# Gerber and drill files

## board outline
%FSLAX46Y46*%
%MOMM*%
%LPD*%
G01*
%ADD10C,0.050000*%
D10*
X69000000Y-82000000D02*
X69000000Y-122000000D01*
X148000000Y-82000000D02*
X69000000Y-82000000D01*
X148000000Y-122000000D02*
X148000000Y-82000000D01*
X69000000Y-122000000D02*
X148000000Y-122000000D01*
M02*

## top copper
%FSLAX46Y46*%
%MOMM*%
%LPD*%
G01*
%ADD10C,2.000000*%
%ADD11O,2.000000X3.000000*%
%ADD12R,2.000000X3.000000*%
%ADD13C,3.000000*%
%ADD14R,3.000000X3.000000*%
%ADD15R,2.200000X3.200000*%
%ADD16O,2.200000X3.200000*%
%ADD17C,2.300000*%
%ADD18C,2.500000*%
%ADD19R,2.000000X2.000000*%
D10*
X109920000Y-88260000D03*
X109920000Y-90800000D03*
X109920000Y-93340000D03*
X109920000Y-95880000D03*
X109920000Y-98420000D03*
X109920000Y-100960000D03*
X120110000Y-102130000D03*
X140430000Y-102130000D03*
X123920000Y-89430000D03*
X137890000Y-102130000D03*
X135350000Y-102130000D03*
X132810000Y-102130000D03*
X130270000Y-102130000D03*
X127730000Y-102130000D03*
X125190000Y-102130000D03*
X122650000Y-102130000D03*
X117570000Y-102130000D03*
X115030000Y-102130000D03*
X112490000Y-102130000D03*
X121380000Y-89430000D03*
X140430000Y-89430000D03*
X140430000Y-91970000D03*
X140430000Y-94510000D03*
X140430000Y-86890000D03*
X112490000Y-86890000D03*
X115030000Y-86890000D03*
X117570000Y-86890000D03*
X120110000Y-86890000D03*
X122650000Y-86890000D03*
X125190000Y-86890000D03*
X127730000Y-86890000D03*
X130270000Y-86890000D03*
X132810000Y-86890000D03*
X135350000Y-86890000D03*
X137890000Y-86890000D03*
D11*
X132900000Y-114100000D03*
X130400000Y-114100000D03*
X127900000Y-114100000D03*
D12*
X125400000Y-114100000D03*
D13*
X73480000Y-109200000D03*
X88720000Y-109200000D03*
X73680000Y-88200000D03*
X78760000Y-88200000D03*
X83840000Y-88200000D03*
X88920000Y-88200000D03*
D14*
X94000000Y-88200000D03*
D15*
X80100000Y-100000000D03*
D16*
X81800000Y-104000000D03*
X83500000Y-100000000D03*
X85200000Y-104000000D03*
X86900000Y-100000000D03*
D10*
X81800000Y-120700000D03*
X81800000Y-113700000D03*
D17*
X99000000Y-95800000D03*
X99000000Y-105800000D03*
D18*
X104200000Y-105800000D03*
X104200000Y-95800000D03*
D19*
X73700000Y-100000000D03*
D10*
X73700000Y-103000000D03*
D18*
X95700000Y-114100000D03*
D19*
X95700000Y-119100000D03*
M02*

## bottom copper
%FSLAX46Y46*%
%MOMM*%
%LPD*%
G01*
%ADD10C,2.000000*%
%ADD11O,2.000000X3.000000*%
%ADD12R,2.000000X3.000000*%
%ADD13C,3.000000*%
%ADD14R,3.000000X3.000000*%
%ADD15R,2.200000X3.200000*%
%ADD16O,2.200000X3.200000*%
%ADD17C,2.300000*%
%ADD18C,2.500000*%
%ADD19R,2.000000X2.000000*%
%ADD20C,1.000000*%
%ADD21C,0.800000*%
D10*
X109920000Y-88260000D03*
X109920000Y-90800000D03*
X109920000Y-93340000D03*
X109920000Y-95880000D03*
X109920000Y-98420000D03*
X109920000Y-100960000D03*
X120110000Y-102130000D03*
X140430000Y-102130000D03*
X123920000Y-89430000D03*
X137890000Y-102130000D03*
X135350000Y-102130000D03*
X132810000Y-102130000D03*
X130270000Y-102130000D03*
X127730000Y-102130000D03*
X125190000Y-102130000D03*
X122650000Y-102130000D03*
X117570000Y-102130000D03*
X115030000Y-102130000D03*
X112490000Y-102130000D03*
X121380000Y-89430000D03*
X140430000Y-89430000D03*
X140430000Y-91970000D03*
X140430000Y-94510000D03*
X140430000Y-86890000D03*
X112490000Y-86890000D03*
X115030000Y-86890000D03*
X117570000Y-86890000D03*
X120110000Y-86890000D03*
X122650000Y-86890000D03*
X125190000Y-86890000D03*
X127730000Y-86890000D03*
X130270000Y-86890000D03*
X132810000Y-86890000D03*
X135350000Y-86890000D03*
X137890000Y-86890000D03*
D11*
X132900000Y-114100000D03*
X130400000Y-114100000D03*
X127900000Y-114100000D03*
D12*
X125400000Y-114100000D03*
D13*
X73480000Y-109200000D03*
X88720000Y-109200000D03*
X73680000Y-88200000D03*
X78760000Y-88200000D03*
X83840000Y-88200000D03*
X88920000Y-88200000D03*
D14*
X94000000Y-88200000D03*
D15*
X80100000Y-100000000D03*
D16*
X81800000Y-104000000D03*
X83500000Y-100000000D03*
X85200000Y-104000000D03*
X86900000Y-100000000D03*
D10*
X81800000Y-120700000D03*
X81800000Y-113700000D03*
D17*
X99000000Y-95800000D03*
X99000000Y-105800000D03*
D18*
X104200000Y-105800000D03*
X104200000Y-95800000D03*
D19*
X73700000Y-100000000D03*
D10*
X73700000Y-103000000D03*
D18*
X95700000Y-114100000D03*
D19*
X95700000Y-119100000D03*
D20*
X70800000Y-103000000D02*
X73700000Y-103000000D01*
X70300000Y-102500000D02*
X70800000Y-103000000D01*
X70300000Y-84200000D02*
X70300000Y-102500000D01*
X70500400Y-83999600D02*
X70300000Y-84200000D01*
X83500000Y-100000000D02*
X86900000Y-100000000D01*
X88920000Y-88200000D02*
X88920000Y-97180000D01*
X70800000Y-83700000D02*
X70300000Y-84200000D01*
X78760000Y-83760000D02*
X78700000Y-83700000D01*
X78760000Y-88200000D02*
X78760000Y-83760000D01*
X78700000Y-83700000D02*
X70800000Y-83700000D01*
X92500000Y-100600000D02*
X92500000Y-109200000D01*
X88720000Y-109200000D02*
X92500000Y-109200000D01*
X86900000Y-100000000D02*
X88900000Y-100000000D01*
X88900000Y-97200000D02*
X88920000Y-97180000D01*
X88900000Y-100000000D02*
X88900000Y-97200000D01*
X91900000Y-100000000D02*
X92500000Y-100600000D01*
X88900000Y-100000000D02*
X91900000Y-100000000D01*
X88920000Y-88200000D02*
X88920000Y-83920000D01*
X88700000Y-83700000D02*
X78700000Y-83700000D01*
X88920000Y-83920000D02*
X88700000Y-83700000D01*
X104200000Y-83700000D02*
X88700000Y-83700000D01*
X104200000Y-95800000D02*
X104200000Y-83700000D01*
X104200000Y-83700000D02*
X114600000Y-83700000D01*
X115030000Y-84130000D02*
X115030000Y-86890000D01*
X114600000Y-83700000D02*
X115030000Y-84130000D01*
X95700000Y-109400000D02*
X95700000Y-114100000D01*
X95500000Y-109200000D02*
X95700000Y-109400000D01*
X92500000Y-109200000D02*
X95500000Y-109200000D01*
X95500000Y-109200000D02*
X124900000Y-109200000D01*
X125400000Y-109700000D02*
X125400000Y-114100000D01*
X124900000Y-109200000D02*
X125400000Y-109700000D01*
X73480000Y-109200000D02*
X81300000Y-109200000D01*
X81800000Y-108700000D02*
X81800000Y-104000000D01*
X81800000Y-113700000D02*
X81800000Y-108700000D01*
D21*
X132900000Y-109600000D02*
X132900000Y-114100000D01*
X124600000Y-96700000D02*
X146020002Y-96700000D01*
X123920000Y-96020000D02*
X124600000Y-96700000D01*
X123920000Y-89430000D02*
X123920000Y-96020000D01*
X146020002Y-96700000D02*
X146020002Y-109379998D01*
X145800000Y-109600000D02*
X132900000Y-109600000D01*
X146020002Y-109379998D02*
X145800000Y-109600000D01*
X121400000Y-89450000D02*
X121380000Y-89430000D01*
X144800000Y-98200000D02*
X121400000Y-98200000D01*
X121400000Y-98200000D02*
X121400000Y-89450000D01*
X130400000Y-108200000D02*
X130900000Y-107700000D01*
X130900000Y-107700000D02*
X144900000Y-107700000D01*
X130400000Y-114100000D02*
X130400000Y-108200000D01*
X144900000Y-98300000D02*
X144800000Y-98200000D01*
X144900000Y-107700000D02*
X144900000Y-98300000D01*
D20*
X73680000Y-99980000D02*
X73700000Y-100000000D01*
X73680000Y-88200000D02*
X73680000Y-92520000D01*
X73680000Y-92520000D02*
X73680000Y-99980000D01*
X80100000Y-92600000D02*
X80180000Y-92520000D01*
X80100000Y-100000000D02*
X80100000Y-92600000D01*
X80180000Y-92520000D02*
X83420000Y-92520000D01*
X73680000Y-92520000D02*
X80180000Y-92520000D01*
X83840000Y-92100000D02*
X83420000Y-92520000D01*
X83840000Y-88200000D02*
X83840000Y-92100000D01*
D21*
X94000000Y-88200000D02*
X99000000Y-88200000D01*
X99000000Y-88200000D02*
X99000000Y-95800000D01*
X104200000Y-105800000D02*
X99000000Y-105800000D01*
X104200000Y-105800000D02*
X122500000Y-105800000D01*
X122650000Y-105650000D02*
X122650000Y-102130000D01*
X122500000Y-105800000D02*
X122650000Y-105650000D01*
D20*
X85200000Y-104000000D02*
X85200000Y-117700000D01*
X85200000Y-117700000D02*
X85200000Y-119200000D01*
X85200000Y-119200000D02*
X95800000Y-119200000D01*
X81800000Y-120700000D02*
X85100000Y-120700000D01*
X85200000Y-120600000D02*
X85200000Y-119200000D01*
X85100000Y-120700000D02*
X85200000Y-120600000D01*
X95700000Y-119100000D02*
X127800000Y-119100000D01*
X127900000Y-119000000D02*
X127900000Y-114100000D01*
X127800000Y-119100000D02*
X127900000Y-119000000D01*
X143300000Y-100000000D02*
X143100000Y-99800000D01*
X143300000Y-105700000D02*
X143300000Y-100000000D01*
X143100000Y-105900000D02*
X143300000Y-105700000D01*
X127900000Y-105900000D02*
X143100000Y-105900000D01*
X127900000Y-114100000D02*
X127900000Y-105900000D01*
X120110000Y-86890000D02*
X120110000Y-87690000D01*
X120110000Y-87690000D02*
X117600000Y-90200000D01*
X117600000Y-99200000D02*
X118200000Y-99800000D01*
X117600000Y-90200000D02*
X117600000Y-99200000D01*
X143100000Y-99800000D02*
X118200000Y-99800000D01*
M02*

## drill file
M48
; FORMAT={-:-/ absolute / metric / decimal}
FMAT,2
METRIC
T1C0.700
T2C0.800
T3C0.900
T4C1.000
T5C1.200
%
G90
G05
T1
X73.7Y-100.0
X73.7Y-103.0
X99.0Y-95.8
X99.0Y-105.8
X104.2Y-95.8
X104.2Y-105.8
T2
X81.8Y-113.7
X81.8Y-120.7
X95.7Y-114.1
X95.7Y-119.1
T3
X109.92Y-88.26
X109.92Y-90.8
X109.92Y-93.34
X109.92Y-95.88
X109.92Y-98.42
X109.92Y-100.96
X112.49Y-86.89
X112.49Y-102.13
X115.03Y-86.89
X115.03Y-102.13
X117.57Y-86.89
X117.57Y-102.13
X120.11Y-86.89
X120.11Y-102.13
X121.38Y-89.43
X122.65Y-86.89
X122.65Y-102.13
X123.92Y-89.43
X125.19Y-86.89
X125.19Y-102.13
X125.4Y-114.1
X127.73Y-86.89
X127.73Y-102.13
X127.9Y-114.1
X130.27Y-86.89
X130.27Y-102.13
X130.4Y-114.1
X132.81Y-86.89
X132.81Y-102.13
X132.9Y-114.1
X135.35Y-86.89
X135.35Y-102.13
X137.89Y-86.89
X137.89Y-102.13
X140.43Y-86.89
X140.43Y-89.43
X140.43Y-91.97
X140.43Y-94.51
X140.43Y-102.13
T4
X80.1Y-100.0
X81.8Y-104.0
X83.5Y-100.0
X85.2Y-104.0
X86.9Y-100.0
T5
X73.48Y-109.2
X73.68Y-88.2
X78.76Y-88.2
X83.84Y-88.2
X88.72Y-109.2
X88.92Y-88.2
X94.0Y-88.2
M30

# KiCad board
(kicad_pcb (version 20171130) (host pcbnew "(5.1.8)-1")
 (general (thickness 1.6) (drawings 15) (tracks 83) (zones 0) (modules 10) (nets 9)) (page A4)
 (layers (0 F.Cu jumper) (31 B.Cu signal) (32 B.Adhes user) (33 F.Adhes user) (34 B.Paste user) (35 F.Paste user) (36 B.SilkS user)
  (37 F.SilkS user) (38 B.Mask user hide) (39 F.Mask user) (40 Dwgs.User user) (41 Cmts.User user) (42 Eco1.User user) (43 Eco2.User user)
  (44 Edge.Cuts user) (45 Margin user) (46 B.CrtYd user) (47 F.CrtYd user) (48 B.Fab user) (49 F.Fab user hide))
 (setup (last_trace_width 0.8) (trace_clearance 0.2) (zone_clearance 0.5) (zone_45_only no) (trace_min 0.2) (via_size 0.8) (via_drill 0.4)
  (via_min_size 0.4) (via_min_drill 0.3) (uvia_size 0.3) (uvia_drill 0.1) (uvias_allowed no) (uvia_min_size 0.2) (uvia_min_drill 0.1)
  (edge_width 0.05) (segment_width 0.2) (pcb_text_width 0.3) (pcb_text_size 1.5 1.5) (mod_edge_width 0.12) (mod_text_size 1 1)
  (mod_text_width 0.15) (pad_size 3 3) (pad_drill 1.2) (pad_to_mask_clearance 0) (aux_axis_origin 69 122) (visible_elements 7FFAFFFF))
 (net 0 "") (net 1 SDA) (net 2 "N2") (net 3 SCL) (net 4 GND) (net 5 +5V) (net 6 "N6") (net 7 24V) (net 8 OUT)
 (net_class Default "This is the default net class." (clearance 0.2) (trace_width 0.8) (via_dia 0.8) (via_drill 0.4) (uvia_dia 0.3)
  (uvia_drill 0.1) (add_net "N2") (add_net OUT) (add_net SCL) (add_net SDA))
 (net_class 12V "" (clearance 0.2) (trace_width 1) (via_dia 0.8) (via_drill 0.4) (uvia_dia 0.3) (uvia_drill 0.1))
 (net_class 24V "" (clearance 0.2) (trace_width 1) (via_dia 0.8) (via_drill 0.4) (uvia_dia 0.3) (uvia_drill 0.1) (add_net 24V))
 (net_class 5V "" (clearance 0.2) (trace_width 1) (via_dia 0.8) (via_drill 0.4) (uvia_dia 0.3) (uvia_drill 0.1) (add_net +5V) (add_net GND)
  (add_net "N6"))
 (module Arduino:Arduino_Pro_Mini (layer F.Cu) (at 141.7 103.4 90)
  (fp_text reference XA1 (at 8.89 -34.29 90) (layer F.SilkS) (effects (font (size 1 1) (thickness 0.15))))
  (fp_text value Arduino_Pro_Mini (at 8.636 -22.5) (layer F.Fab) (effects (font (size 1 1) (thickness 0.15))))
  (pad GND5 thru_hole circle (at 15.14 -31.78 90) (size 2 2) (drill 0.9) (layers *.Cu *.Mask))
  (pad GND4 thru_hole circle (at 12.6 -31.78 90) (size 2 2) (drill 0.9) (layers *.Cu *.Mask))
  (pad VCC1 thru_hole circle (at 10.06 -31.78 90) (size 2 2) (drill 0.9) (layers *.Cu *.Mask))
  (pad RXI thru_hole circle (at 7.52 -31.78 90) (size 2 2) (drill 0.9) (layers *.Cu *.Mask))
  (pad TX0 thru_hole circle (at 4.98 -31.78 90) (size 2 2) (drill 0.9) (layers *.Cu *.Mask))
  (pad DTR thru_hole circle (at 2.44 -31.78 90) (size 2 2) (drill 0.9) (layers *.Cu *.Mask))
  (pad GND2 thru_hole circle (at 1.27 -21.59 90) (size 2 2) (drill 0.9) (layers *.Cu *.Mask))
  (pad D9 thru_hole circle (at 1.27 -1.27 90) (size 2 2) (drill 0.9) (layers *.Cu *.Mask))
  (pad A4 thru_hole circle (at 13.97 -17.78 90) (size 2 2) (drill 0.9) (layers *.Cu *.Mask) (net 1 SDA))
  (pad D8 thru_hole circle (at 1.27 -3.81 90) (size 2 2) (drill 0.9) (layers *.Cu *.Mask))
  (pad D7 thru_hole circle (at 1.27 -6.35 90) (size 2 2) (drill 0.9) (layers *.Cu *.Mask))
  (pad D6 thru_hole circle (at 1.27 -8.89 90) (size 2 2) (drill 0.9) (layers *.Cu *.Mask))
  (pad D5 thru_hole circle (at 1.27 -11.43 90) (size 2 2) (drill 0.9) (layers *.Cu *.Mask))
  (pad D4 thru_hole circle (at 1.27 -13.97 90) (size 2 2) (drill 0.9) (layers *.Cu *.Mask))
  (pad D3 thru_hole circle (at 1.27 -16.51 90) (size 2 2) (drill 0.9) (layers *.Cu *.Mask))
  (pad D2 thru_hole circle (at 1.27 -19.05 90) (size 2 2) (drill 0.9) (layers *.Cu *.Mask) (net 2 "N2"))
  (pad RST2 thru_hole circle (at 1.27 -24.13 90) (size 2 2) (drill 0.9) (layers *.Cu *.Mask))
  (pad D1 thru_hole circle (at 1.27 -26.67 90) (size 2 2) (drill 0.9) (layers *.Cu *.Mask))
  (pad D0 thru_hole circle (at 1.27 -29.21 90) (size 2 2) (drill 0.9) (layers *.Cu *.Mask))
  (pad A5 thru_hole circle (at 13.97 -20.32 90) (size 2 2) (drill 0.9) (layers *.Cu *.Mask) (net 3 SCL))
  (pad A7 thru_hole circle (at 13.97 -1.27 90) (size 2 2) (drill 0.9) (layers *.Cu *.Mask))
  (pad A6 thru_hole circle (at 11.43 -1.27 90) (size 2 2) (drill 0.9) (layers *.Cu *.Mask))
  (pad GND3 thru_hole circle (at 8.89 -1.27 90) (size 2 2) (drill 0.9) (layers *.Cu *.Mask))
  (pad D10 thru_hole circle (at 16.51 -1.27 90) (size 2 2) (drill 0.9) (layers *.Cu *.Mask))
  (pad RAW thru_hole circle (at 16.51 -29.21 90) (size 2 2) (drill 0.9) (layers *.Cu *.Mask))
  (pad GND thru_hole circle (at 16.51 -26.67 90) (size 2 2) (drill 0.9) (layers *.Cu *.Mask) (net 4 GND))
  (pad RST thru_hole circle (at 16.51 -24.13 90) (size 2 2) (drill 0.9) (layers *.Cu *.Mask))
  (pad VCC thru_hole circle (at 16.51 -21.59 90) (size 2 2) (drill 0.9) (layers *.Cu *.Mask) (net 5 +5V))
  (pad A3 thru_hole circle (at 16.51 -19.05 90) (size 2 2) (drill 0.9) (layers *.Cu *.Mask))
  (pad A2 thru_hole circle (at 16.51 -16.51 90) (size 2 2) (drill 0.9) (layers *.Cu *.Mask))
  (pad A1 thru_hole circle (at 16.51 -13.97 90) (size 2 2) (drill 0.9) (layers *.Cu *.Mask))
  (pad A0 thru_hole circle (at 16.51 -11.43 90) (size 2 2) (drill 0.9) (layers *.Cu *.Mask))
  (pad D13 thru_hole circle (at 16.51 -8.89 90) (size 2 2) (drill 0.9) (layers *.Cu *.Mask))
  (pad D12 thru_hole circle (at 16.51 -6.35 90) (size 2 2) (drill 0.9) (layers *.Cu *.Mask))
  (pad D11 thru_hole circle (at 16.51 -3.81 90) (size 2 2) (drill 0.9) (layers *.Cu *.Mask)))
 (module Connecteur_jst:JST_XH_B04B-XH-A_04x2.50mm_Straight (layer F.Cu) (at 125.4 114.1)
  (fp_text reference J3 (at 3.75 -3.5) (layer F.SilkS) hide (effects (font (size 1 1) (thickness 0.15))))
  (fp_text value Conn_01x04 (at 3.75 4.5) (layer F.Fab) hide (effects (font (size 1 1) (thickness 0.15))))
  (pad 4 thru_hole oval (at 7.5 0) (size 2 3) (drill 0.9) (layers *.Cu *.Mask) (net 1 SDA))
  (pad 3 thru_hole oval (at 5 0) (size 2 3) (drill 0.9) (layers *.Cu *.Mask) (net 3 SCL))
  (pad 2 thru_hole oval (at 2.5 0) (size 2 3) (drill 0.9) (layers *.Cu *.Mask) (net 5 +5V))
  (pad 1 thru_hole rect (at 0 0) (size 2 3) (drill 0.9) (layers *.Cu *.Mask) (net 4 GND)))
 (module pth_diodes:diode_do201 (layer F.Cu) (at 81.1 109.2 180)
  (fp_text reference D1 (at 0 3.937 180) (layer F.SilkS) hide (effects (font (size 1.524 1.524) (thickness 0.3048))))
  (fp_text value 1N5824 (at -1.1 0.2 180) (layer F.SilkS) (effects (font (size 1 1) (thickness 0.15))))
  (pad 1 thru_hole circle (at 7.62 0 180) (size 3 3) (drill 1.2) (layers *.Cu *.Mask) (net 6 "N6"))
  (pad 2 thru_hole circle (at -7.62 0 180) (size 3 3) (drill 1.2) (layers *.Cu *.Mask) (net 4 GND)))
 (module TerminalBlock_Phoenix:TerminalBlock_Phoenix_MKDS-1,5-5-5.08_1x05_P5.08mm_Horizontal (layer F.Cu) (at 94 88.2 180)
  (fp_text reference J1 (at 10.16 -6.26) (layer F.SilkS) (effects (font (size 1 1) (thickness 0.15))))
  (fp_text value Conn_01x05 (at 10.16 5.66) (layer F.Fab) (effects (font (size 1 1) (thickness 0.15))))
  (pad 5 thru_hole circle (at 20.32 0 180) (size 3 3) (drill 1.2) (layers *.Cu *.Mask) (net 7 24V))
  (pad 4 thru_hole circle (at 15.24 0 180) (size 3 3) (drill 1.2) (layers *.Cu *.Mask) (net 4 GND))
  (pad 3 thru_hole circle (at 10.16 0 180) (size 3 3) (drill 1.2) (layers *.Cu *.Mask) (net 7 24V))
  (pad 2 thru_hole circle (at 5.08 0 180) (size 3 3) (drill 1.2) (layers *.Cu *.Mask) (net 4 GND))
  (pad 1 thru_hole rect (at 0 0 180) (size 3 3) (drill 1.2) (layers *.Cu *.Mask) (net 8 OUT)))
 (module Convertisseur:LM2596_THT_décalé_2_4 (layer F.Cu) (at 80.1 100)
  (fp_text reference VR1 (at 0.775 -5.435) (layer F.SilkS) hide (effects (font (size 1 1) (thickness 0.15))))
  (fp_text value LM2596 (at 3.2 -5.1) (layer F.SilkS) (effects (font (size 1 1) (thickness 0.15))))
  (pad 1 thru_hole rect (at 0 0) (size 2.2 3.2) (drill 1) (layers *.Cu *.Mask) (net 7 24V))
  (pad 2 thru_hole oval (at 1.7 4) (size 2.2 3.2) (drill 1) (layers *.Cu *.Mask) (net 6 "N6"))
  (pad 3 thru_hole oval (at 3.4 0) (size 2.2 3.2) (drill 1) (layers *.Cu *.Mask) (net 4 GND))
  (pad 4 thru_hole oval (at 5.1 4) (size 2.2 3.2) (drill 1) (layers *.Cu *.Mask) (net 5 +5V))
  (pad 5 thru_hole oval (at 6.8 0) (size 2.2 3.2) (drill 1) (layers *.Cu *.Mask) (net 4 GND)))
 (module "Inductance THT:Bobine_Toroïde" (layer F.Cu) (at 81.8 117.7)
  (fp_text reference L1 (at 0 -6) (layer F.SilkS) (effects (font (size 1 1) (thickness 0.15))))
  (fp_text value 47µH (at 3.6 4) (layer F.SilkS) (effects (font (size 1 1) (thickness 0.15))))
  (pad 2 thru_hole circle (at 0 3) (size 2 2) (drill 0.8) (layers *.Cu *.Mask) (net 5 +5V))
  (pad 1 thru_hole circle (at 0 -4) (size 2 2) (drill 0.8) (layers *.Cu *.Mask) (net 6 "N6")))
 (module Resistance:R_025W (layer F.Cu) (at 99.1 100.9 270) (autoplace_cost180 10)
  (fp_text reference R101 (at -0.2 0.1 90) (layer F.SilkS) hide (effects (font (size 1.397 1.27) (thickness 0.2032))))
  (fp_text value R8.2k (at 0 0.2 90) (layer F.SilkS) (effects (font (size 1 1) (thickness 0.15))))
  (pad 1 thru_hole circle (at -5.1 0.1 270) (size 2.3 2.3) (drill 0.7) (layers *.Cu *.Mask) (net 8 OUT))
  (pad 2 thru_hole circle (at 4.9 0.1 270) (size 2.3 2.3) (drill 0.7) (layers *.Cu *.Mask) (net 2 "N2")))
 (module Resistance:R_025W (layer F.Cu) (at 104.1 100.7 90) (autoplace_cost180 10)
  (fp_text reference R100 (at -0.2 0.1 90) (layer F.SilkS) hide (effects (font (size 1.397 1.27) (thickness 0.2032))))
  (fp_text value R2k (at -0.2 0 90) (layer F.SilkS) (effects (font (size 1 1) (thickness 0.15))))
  (pad 1 thru_hole circle (at -5.1 0.1 90) (size 2.5 2.5) (drill 0.7) (layers *.Cu *.Mask) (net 2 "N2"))
  (pad 2 thru_hole circle (at 4.9 0.1 90) (size 2.5 2.5) (drill 0.7) (layers *.Cu *.Mask) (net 4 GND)))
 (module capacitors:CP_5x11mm (layer F.Cu) (at 73.7 101.5 180)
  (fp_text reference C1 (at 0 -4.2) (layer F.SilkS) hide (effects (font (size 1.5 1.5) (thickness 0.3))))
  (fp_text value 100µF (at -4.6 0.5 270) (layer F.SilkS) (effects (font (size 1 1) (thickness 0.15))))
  (pad 1 thru_hole rect (at 0 1.5 180) (size 2 2) (drill 0.7) (layers *.Cu F.Mask) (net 7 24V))
  (pad 2 thru_hole circle (at 0 -1.5 180) (size 2 2) (drill 0.7) (layers *.Cu *.Mask) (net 4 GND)))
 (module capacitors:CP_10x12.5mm (layer F.Cu) (at 95.7 116.6)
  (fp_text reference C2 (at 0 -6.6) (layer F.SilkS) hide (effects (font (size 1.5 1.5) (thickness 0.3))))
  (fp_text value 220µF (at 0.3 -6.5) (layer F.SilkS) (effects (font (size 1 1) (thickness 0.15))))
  (pad 2 thru_hole circle (at 0 -2.5) (size 2.5 2.5) (drill 0.8) (layers *.Cu *.Mask) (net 4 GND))
  (pad 1 thru_hole rect (at 0 2.5) (size 2 2) (drill 0.8) (layers *.Cu *.Mask) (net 5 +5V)))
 (gr_line (start 69 82) (end 69 122) (layer Edge.Cuts) (width 0.05))
 (gr_line (start 148 82) (end 69 82) (layer Edge.Cuts) (width 0.05))
 (gr_line (start 148 122) (end 148 82) (layer Edge.Cuts) (width 0.05))
 (gr_line (start 69 122) (end 148 122) (layer Edge.Cuts) (width 0.05))
 (segment (start 70.8 103) (end 73.7 103) (width 1) (layer B.Cu) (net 4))
 (segment (start 70.3 102.5) (end 70.8 103) (width 1) (layer B.Cu) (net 4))
 (segment (start 70.3 84.2) (end 70.3 102.5) (width 1) (layer B.Cu) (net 4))
 (segment (start 70.5004 83.9996) (end 70.3 84.2) (width 1) (layer B.Cu) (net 4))
 (segment (start 83.5 100) (end 86.9 100) (width 1) (layer B.Cu) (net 4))
 (segment (start 88.92 88.2) (end 88.92 97.18) (width 1) (layer B.Cu) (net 4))
 (segment (start 70.8 83.7) (end 70.3 84.2) (width 1) (layer B.Cu) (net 4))
 (segment (start 78.76 83.76) (end 78.7 83.7) (width 1) (layer B.Cu) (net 4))
 (segment (start 78.76 88.2) (end 78.76 83.76) (width 1) (layer B.Cu) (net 4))
 (segment (start 78.7 83.7) (end 70.8 83.7) (width 1) (layer B.Cu) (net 4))
 (segment (start 92.5 100.6) (end 92.5 109.2) (width 1) (layer B.Cu) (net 4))
 (segment (start 88.72 109.2) (end 92.5 109.2) (width 1) (layer B.Cu) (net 4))
 (segment (start 86.9 100) (end 88.9 100) (width 1) (layer B.Cu) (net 4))
 (segment (start 88.9 97.2) (end 88.92 97.18) (width 1) (layer B.Cu) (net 4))
 (segment (start 88.9 100) (end 88.9 97.2) (width 1) (layer B.Cu) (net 4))
 (segment (start 91.9 100) (end 92.5 100.6) (width 1) (layer B.Cu) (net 4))
 (segment (start 88.9 100) (end 91.9 100) (width 1) (layer B.Cu) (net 4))
 (segment (start 88.92 88.2) (end 88.92 83.92) (width 1) (layer B.Cu) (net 4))
 (segment (start 88.7 83.7) (end 78.7 83.7) (width 1) (layer B.Cu) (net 4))
 (segment (start 88.92 83.92) (end 88.7 83.7) (width 1) (layer B.Cu) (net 4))
 (segment (start 104.2 83.7) (end 88.7 83.7) (width 1) (layer B.Cu) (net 4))
 (segment (start 104.2 95.8) (end 104.2 83.7) (width 1) (layer B.Cu) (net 4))
 (segment (start 104.2 83.7) (end 114.6 83.7) (width 1) (layer B.Cu) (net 4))
 (segment (start 115.03 84.13) (end 115.03 86.89) (width 1) (layer B.Cu) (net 4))
 (segment (start 114.6 83.7) (end 115.03 84.13) (width 1) (layer B.Cu) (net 4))
 (segment (start 95.7 109.4) (end 95.7 114.1) (width 1) (layer B.Cu) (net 4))
 (segment (start 95.5 109.2) (end 95.7 109.4) (width 1) (layer B.Cu) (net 4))
 (segment (start 92.5 109.2) (end 95.5 109.2) (width 1) (layer B.Cu) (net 4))
 (segment (start 95.5 109.2) (end 124.9 109.2) (width 1) (layer B.Cu) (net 4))
 (segment (start 125.4 109.7) (end 125.4 114.1) (width 1) (layer B.Cu) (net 4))
 (segment (start 124.9 109.2) (end 125.4 109.7) (width 1) (layer B.Cu) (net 4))
 (segment (start 73.48 109.2) (end 81.3 109.2) (width 1) (layer B.Cu) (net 6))
 (segment (start 81.8 108.7) (end 81.8 104) (width 1) (layer B.Cu) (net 6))
 (segment (start 81.8 113.7) (end 81.8 108.7) (width 1) (layer B.Cu) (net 6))
 (segment (start 132.9 109.6) (end 132.9 114.1) (width 0.8) (layer B.Cu) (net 1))
 (segment (start 124.6 96.7) (end 146.020002 96.7) (width 0.8) (layer B.Cu) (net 1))
 (segment (start 123.92 96.02) (end 124.6 96.7) (width 0.8) (layer B.Cu) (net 1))
 (segment (start 123.92 89.43) (end 123.92 96.02) (width 0.8) (layer B.Cu) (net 1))
 (segment (start 146.020002 96.7) (end 146.020002 109.379998) (width 0.8) (layer B.Cu) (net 1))
 (segment (start 145.8 109.6) (end 132.9 109.6) (width 0.8) (layer B.Cu) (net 1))
 (segment (start 146.020002 109.379998) (end 145.8 109.6) (width 0.8) (layer B.Cu) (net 1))
 (segment (start 121.4 89.45) (end 121.38 89.43) (width 0.8) (layer B.Cu) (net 3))
 (segment (start 144.8 98.2) (end 121.4 98.2) (width 0.8) (layer B.Cu) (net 3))
 (segment (start 121.4 98.2) (end 121.4 89.45) (width 0.8) (layer B.Cu) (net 3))
 (segment (start 130.4 108.2) (end 130.9 107.7) (width 0.8) (layer B.Cu) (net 3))
 (segment (start 130.9 107.7) (end 144.9 107.7) (width 0.8) (layer B.Cu) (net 3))
 (segment (start 130.4 114.1) (end 130.4 108.2) (width 0.8) (layer B.Cu) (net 3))
 (segment (start 144.9 98.3) (end 144.8 98.2) (width 0.8) (layer B.Cu) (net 3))
 (segment (start 144.9 107.7) (end 144.9 98.3) (width 0.8) (layer B.Cu) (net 3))
 (segment (start 73.68 99.98) (end 73.7 100) (width 1) (layer B.Cu) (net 7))
 (segment (start 73.68 88.2) (end 73.68 92.52) (width 1) (layer B.Cu) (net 7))
 (segment (start 73.68 92.52) (end 73.68 99.98) (width 1) (layer B.Cu) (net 7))
 (segment (start 80.1 92.6) (end 80.18 92.52) (width 1) (layer B.Cu) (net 7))
 (segment (start 80.1 100) (end 80.1 92.6) (width 1) (layer B.Cu) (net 7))
 (segment (start 80.18 92.52) (end 83.42 92.52) (width 1) (layer B.Cu) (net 7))
 (segment (start 73.68 92.52) (end 80.18 92.52) (width 1) (layer B.Cu) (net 7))
 (segment (start 83.84 92.1) (end 83.42 92.52) (width 1) (layer B.Cu) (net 7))
 (segment (start 83.84 88.2) (end 83.84 92.1) (width 1) (layer B.Cu) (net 7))
 (segment (start 94 88.2) (end 99 88.2) (width 0.8) (layer B.Cu) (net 8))
 (segment (start 99 88.2) (end 99 95.8) (width 0.8) (layer B.Cu) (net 8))
 (segment (start 104.2 105.8) (end 99 105.8) (width 0.8) (layer B.Cu) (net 2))
 (segment (start 104.2 105.8) (end 122.5 105.8) (width 0.8) (layer B.Cu) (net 2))
 (segment (start 122.65 105.65) (end 122.65 102.13) (width 0.8) (layer B.Cu) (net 2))
 (segment (start 122.5 105.8) (end 122.65 105.65) (width 0.8) (layer B.Cu) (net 2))
 (segment (start 85.2 104) (end 85.2 117.7) (width 1) (layer B.Cu) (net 5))
 (segment (start 85.2 117.7) (end 85.2 119.2) (width 1) (layer B.Cu) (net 5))
 (segment (start 85.2 119.2) (end 95.8 119.2) (width 1) (layer B.Cu) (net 5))
 (segment (start 81.8 120.7) (end 85.1 120.7) (width 1) (layer B.Cu) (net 5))
 (segment (start 85.2 120.6) (end 85.2 119.2) (width 1) (layer B.Cu) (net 5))
 (segment (start 85.1 120.7) (end 85.2 120.6) (width 1) (layer B.Cu) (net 5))
 (segment (start 95.7 119.1) (end 127.8 119.1) (width 1) (layer B.Cu) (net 5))
 (segment (start 127.9 119) (end 127.9 114.1) (width 1) (layer B.Cu) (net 5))
 (segment (start 127.8 119.1) (end 127.9 119) (width 1) (layer B.Cu) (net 5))
 (segment (start 143.3 100) (end 143.1 99.8) (width 1) (layer B.Cu) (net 5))
 (segment (start 143.3 105.7) (end 143.3 100) (width 1) (layer B.Cu) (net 5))
 (segment (start 143.1 105.9) (end 143.3 105.7) (width 1) (layer B.Cu) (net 5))
 (segment (start 127.9 105.9) (end 143.1 105.9) (width 1) (layer B.Cu) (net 5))
 (segment (start 127.9 114.1) (end 127.9 105.9) (width 1) (layer B.Cu) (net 5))
 (segment (start 120.11 86.89) (end 120.11 87.69) (width 1) (layer B.Cu) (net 5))
 (segment (start 120.11 87.69) (end 117.6 90.2) (width 1) (layer B.Cu) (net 5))
 (segment (start 117.6 99.2) (end 118.2 99.8) (width 1) (layer B.Cu) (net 5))
 (segment (start 117.6 90.2) (end 117.6 99.2) (width 1) (layer B.Cu) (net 5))
 (segment (start 143.1 99.8) (end 118.2 99.8) (width 1) (layer B.Cu) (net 5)))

